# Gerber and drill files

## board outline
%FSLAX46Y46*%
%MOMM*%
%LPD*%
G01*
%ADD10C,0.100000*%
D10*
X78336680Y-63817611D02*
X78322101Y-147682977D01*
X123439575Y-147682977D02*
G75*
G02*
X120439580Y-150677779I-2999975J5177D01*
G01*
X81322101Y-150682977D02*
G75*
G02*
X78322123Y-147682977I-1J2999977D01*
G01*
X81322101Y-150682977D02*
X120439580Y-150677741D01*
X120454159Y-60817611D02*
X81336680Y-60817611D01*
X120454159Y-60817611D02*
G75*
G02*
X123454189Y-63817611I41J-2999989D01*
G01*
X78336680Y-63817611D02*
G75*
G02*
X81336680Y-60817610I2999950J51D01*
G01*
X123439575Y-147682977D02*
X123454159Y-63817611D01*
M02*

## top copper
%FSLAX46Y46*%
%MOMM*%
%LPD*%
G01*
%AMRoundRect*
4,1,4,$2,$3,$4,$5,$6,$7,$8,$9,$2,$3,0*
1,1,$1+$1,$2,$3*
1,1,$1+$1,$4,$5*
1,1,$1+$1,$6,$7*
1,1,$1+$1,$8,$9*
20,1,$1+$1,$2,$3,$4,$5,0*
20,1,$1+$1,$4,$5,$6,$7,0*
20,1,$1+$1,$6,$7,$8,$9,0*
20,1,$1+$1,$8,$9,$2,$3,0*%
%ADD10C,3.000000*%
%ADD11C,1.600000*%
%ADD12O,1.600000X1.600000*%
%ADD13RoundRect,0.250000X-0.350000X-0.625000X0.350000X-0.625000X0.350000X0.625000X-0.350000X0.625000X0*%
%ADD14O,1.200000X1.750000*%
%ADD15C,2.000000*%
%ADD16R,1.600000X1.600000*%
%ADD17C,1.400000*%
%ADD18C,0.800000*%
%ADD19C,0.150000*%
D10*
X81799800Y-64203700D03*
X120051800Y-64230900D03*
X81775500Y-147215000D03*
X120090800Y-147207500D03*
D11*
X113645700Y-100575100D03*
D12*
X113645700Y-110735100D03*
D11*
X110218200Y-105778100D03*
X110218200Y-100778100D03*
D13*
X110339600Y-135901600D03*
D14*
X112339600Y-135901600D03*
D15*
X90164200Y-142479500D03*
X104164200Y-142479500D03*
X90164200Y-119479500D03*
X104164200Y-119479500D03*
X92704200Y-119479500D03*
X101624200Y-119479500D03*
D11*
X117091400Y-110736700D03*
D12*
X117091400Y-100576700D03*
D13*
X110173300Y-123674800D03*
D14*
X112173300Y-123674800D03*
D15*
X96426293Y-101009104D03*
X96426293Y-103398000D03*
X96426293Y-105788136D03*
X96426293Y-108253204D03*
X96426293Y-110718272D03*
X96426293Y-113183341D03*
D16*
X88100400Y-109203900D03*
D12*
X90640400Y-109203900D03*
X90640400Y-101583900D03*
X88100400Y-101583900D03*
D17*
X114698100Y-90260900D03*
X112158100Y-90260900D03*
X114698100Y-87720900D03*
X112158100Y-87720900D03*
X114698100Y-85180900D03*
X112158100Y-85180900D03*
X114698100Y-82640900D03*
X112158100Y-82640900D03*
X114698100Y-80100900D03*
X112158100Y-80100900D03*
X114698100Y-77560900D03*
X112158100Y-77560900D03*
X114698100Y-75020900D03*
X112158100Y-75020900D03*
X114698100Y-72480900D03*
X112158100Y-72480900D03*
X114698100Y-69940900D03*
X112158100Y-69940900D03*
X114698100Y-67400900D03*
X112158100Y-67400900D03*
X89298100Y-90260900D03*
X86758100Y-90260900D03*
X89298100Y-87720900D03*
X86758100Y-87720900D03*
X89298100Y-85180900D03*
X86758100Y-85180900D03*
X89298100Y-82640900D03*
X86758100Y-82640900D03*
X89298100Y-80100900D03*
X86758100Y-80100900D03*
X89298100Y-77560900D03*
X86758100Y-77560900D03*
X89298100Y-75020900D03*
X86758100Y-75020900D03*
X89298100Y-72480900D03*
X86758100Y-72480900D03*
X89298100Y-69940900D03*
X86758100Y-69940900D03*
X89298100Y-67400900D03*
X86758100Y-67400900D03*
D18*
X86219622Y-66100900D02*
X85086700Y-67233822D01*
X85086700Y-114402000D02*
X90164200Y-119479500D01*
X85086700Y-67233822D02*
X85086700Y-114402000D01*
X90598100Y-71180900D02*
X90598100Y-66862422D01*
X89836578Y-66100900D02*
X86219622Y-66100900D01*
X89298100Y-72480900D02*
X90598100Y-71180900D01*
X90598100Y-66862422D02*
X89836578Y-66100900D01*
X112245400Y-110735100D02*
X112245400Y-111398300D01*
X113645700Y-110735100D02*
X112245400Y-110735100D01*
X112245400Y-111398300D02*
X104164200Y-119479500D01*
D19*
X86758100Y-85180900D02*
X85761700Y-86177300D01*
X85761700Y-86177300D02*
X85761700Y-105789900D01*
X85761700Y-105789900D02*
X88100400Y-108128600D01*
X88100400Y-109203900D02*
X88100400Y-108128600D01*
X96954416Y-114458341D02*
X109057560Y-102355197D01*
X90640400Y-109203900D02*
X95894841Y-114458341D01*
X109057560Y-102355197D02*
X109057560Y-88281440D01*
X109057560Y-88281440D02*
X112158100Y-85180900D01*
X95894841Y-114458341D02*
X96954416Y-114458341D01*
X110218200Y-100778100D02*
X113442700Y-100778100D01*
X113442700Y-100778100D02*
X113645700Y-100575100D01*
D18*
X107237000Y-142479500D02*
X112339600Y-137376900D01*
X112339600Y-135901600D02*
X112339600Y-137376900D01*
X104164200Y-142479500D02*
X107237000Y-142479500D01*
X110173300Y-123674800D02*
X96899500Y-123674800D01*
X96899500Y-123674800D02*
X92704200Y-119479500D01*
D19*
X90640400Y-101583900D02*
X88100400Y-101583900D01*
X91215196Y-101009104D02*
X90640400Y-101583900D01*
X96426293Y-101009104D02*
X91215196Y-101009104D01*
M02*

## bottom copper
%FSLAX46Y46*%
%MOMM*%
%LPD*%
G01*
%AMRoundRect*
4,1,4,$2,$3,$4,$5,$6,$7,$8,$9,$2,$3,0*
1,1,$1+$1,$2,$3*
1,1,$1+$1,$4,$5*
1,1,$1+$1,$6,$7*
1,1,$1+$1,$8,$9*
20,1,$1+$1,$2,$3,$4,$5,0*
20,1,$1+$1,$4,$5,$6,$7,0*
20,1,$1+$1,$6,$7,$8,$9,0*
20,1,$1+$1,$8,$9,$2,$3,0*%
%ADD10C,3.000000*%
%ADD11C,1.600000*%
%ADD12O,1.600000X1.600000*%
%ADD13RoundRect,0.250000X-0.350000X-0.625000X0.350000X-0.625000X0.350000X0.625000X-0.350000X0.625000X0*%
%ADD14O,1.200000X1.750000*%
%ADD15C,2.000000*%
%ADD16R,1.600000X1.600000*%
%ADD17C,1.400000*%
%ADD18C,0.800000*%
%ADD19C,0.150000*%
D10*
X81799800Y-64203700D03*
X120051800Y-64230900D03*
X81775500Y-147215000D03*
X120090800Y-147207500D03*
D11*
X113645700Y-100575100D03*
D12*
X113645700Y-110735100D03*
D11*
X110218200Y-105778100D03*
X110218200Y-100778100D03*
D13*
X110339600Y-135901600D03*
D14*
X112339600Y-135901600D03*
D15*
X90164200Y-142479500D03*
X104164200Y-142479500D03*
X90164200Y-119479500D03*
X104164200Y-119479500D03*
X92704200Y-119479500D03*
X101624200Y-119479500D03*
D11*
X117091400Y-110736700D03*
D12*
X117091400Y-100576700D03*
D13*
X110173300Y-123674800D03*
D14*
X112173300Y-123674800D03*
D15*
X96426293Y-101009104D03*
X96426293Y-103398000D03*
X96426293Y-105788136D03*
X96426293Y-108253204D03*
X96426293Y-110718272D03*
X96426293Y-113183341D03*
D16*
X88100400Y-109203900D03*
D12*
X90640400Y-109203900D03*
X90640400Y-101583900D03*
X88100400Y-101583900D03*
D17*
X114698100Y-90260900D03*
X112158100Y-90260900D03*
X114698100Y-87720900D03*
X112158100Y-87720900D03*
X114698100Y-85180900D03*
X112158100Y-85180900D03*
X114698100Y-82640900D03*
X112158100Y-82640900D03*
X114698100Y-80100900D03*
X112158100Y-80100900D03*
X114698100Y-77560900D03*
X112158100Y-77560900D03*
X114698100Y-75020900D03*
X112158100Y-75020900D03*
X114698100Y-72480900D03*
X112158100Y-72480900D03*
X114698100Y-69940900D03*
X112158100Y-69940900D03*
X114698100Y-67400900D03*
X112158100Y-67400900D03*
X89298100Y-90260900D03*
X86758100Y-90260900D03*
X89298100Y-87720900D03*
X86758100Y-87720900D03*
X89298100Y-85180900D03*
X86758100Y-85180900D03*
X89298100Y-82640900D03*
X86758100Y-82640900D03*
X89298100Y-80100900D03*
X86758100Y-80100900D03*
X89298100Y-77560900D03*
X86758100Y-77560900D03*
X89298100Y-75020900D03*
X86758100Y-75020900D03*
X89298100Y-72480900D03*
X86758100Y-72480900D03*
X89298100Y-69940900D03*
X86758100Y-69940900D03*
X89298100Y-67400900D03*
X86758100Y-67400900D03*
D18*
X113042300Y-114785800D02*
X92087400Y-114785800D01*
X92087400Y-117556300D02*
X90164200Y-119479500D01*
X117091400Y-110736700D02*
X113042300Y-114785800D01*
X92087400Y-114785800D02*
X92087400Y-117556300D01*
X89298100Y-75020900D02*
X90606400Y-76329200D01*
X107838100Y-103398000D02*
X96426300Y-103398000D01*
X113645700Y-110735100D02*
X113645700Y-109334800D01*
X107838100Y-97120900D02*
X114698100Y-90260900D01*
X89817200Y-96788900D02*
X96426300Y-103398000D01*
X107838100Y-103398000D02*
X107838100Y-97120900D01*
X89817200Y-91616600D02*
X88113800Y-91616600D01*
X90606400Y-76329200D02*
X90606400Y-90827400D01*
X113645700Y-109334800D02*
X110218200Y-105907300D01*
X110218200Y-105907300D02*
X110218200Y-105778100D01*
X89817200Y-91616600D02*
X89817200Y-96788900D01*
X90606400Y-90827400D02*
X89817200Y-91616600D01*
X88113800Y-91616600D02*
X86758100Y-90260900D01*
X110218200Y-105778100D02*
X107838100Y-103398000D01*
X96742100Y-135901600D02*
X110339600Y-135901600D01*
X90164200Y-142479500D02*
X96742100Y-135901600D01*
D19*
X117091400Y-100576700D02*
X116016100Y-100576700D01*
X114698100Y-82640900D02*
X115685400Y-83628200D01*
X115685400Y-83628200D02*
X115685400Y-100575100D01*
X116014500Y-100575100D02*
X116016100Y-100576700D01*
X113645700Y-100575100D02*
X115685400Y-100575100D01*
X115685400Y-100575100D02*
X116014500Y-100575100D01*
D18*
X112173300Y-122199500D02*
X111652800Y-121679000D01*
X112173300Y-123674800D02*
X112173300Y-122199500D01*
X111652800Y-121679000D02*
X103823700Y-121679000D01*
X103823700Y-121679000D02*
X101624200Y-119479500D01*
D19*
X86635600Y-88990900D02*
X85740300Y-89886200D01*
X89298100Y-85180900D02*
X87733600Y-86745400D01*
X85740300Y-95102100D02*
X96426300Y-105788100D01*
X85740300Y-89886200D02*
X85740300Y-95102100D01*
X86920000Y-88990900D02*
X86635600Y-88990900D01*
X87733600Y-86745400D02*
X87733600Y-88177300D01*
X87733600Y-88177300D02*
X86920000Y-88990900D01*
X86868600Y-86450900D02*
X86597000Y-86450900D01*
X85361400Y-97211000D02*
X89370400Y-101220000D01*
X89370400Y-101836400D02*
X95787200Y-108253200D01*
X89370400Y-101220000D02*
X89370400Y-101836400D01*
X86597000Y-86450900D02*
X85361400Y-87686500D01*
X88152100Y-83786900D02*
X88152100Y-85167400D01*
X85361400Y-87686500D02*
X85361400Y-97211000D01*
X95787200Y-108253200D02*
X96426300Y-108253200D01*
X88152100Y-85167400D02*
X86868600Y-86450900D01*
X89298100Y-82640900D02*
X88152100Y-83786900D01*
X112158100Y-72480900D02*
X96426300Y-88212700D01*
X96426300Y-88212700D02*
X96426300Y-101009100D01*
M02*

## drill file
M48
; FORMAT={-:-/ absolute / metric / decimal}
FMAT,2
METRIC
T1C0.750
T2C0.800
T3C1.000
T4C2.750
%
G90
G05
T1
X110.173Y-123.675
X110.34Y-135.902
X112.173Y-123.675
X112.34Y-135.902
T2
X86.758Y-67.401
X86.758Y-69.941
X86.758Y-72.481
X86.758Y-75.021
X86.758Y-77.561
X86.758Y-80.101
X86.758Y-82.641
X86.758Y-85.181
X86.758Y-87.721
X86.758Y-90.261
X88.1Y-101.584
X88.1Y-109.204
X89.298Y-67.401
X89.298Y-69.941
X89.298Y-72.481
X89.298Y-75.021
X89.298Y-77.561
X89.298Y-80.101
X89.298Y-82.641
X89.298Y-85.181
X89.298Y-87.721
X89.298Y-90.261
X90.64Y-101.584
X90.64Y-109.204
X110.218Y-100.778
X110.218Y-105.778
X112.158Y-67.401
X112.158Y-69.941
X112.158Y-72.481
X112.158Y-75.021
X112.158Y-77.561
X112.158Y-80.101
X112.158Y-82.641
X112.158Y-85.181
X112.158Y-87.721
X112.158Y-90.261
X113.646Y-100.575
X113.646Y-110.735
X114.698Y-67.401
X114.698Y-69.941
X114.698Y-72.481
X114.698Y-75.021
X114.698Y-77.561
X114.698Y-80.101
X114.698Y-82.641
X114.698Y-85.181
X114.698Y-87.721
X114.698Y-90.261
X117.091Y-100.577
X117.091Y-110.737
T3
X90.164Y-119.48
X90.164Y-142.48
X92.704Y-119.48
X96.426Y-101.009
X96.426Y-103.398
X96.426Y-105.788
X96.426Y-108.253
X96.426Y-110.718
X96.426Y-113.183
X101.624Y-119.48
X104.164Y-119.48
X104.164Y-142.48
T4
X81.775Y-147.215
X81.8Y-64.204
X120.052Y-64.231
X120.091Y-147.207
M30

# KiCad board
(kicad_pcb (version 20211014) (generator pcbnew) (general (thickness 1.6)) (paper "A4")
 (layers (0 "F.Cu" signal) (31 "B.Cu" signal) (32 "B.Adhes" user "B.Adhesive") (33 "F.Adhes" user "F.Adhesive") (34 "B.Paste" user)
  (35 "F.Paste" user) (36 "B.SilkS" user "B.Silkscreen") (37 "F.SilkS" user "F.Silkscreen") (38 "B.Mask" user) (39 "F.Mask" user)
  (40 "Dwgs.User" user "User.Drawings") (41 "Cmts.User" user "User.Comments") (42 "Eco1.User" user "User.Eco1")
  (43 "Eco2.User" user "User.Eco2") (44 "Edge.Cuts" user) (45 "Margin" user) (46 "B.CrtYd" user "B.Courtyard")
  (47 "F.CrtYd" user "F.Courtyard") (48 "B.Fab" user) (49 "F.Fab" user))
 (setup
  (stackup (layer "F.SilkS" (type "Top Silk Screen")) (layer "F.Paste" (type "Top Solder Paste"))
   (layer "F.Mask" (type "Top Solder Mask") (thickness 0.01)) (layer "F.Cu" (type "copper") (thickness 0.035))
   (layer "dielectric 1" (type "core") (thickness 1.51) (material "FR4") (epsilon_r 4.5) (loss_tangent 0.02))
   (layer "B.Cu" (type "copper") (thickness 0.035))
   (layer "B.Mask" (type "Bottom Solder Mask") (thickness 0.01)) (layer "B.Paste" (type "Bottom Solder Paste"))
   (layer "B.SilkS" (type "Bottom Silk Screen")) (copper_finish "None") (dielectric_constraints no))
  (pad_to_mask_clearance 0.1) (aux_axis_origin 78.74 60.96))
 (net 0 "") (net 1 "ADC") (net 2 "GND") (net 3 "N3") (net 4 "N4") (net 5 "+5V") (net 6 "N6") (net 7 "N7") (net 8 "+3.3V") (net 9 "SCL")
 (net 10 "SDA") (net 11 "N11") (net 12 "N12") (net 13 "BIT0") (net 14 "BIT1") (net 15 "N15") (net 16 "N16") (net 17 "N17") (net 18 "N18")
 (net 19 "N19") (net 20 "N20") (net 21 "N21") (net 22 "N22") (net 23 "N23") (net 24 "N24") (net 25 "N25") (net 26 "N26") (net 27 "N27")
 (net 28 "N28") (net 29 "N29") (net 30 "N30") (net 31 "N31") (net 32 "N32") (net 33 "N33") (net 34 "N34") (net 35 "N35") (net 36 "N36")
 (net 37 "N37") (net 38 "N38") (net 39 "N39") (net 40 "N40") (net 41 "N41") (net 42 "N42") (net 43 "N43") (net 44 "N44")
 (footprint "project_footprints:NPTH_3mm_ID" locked (layer "F.Cu") (at 81.7998 64.2037)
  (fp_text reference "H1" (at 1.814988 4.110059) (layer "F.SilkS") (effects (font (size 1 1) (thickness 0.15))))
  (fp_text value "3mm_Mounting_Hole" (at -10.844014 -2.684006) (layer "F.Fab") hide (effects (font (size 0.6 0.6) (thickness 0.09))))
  (pad "" np_thru_hole circle locked (at 0 0) (size 3 3) (drill 2.75) (layers *.Cu *.Mask) (clearance 1.6)))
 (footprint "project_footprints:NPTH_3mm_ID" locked (layer "F.Cu") (at 120.0518 64.2309)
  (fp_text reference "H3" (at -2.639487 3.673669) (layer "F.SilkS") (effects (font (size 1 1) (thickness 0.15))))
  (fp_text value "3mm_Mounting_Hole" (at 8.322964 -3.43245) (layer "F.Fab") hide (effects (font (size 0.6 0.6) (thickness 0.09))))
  (pad "" np_thru_hole circle locked (at 0 0) (size 3 3) (drill 2.75) (layers *.Cu *.Mask) (clearance 1.6)))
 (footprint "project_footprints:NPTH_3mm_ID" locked (layer "F.Cu") (at 81.7755 147.215)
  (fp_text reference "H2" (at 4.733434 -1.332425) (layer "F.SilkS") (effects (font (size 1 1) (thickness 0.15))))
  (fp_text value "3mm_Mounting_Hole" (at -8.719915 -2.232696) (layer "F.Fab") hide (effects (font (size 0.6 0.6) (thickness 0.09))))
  (pad "" np_thru_hole circle locked (at 0 0) (size 3 3) (drill 2.75) (layers *.Cu *.Mask) (clearance 1.6)))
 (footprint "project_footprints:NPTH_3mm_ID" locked (layer "F.Cu") (at 120.0908 147.2075)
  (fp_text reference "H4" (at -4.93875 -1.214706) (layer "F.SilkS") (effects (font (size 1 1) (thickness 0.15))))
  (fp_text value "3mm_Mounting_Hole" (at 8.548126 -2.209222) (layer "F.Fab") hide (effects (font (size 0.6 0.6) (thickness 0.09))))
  (pad "" np_thru_hole circle locked (at 0 0) (size 3 3) (drill 2.75) (layers *.Cu *.Mask) (clearance 1.6)))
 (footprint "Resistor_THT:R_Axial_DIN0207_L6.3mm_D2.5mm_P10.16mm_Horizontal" (layer "F.Cu") (at 113.6457 100.5751 -90)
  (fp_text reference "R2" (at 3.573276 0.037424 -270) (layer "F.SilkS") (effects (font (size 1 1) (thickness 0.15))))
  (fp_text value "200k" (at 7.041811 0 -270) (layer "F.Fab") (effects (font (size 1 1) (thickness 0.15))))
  (pad "1" thru_hole circle (at 0 0 270) (size 1.6 1.6) (drill 0.8) (layers *.Cu *.Mask) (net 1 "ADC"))
  (pad "2" thru_hole oval (at 10.16 0 270) (size 1.6 1.6) (drill 0.8) (layers *.Cu *.Mask) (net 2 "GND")))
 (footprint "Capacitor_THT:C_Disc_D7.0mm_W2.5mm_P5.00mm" (layer "F.Cu") (at 110.2182 105.7781 90)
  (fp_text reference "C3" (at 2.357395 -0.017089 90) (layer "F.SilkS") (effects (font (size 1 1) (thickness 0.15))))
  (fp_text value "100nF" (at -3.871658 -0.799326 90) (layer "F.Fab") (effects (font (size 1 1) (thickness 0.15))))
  (pad "1" thru_hole circle (at 0 0 90) (size 1.6 1.6) (drill 0.8) (layers *.Cu *.Mask) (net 2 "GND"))
  (pad "2" thru_hole circle (at 5 0 90) (size 1.6 1.6) (drill 0.8) (layers *.Cu *.Mask) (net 1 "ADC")))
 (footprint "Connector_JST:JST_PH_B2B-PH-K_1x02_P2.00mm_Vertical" (layer "F.Cu") (at 110.3396 135.9016)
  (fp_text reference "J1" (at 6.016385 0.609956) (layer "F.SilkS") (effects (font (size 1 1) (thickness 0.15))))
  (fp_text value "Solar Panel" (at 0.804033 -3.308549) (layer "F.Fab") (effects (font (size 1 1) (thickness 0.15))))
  (pad "1" thru_hole roundrect (at 0 0) (size 1.2 1.75) (drill 0.75) (layers *.Cu *.Mask) (roundrect_rratio 0.208333) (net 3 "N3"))
  (pad "2" thru_hole oval (at 2 0) (size 1.2 1.75) (drill 0.75) (layers *.Cu *.Mask) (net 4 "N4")))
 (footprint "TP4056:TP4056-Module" (layer "F.Cu") (at 105.7642 144.9795 90)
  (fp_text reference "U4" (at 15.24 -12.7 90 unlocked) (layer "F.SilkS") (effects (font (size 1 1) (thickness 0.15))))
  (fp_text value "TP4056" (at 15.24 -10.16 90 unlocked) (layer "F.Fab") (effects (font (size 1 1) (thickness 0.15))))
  (pad "1" thru_hole circle (at 2.5 -15.6 90) (size 2 2) (drill 1) (layers *.Cu *.Mask) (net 3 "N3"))
  (pad "2" thru_hole circle (at 2.5 -1.6 90) (size 2 2) (drill 1) (layers *.Cu *.Mask) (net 4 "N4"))
  (pad "3" thru_hole circle (at 25.5 -15.6 90) (size 2 2) (drill 1) (layers *.Cu *.Mask) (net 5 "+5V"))
  (pad "4" thru_hole circle (at 25.5 -1.6 90) (size 2 2) (drill 1) (layers *.Cu *.Mask) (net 2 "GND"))
  (pad "5" thru_hole circle (at 25.5 -13.06 90) (size 2 2) (drill 1) (layers *.Cu *.Mask) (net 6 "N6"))
  (pad "6" thru_hole circle (at 25.5 -4.14 90) (size 2 2) (drill 1) (layers *.Cu *.Mask) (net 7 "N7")))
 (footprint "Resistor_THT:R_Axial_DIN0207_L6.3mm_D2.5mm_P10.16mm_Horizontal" (layer "F.Cu") (at 117.0914 110.7367 90)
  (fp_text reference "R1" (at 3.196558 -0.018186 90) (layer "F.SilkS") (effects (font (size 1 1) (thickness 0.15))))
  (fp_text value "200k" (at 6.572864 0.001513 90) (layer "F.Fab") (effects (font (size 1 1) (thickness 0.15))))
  (pad "1" thru_hole circle (at 0 0 90) (size 1.6 1.6) (drill 0.8) (layers *.Cu *.Mask) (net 5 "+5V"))
  (pad "2" thru_hole oval (at 10.16 0 90) (size 1.6 1.6) (drill 0.8) (layers *.Cu *.Mask) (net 1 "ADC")))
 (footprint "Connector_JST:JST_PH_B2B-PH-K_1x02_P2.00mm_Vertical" (layer "F.Cu") (at 110.1733 123.6748)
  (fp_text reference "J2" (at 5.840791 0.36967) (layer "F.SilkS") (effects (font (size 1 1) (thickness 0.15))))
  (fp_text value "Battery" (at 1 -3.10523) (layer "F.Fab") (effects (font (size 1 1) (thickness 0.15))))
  (pad "1" thru_hole roundrect (at 0 0) (size 1.2 1.75) (drill 0.75) (layers *.Cu *.Mask) (roundrect_rratio 0.208333) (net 6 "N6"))
  (pad "2" thru_hole oval (at 2 0) (size 1.2 1.75) (drill 0.75) (layers *.Cu *.Mask) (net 7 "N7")))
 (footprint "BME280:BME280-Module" (layer "F.Cu") (at 94.9375 114.558)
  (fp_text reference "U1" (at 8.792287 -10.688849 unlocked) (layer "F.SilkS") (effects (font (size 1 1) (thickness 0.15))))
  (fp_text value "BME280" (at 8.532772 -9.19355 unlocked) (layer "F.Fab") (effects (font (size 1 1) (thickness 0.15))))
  (pad "1" thru_hole circle (at 1.488793 -13.548896) (size 2 2) (drill 1) (layers *.Cu *.Mask) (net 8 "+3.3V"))
  (pad "2" thru_hole circle (at 1.488793 -11.16) (size 2 2) (drill 1) (layers *.Cu *.Mask) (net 2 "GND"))
  (pad "3" thru_hole circle (at 1.488793 -8.769864) (size 2 2) (drill 1) (layers *.Cu *.Mask) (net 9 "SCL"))
  (pad "4" thru_hole circle (at 1.488793 -6.304796) (size 2 2) (drill 1) (layers *.Cu *.Mask) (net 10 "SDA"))
  (pad "5" thru_hole circle (at 1.488793 -3.839728) (size 2 2) (drill 1) (layers *.Cu *.Mask) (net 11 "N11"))
  (pad "6" thru_hole circle (at 1.488793 -1.374659) (size 2 2) (drill 1) (layers *.Cu *.Mask) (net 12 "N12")))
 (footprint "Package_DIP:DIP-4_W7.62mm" (layer "F.Cu") (at 88.1004 109.2039 90)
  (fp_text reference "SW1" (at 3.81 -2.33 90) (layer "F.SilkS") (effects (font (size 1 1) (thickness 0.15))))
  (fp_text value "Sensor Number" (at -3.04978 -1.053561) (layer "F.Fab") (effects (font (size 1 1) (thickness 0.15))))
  (pad "1" thru_hole rect (at 0 0 90) (size 1.6 1.6) (drill 0.8) (layers *.Cu *.Mask) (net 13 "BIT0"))
  (pad "2" thru_hole oval (at 0 2.54 90) (size 1.6 1.6) (drill 0.8) (layers *.Cu *.Mask) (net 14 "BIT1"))
  (pad "3" thru_hole oval (at 7.62 2.54 90) (size 1.6 1.6) (drill 0.8) (layers *.Cu *.Mask) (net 8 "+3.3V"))
  (pad "4" thru_hole oval (at 7.62 0 90) (size 1.6 1.6) (drill 0.8) (layers *.Cu *.Mask) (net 8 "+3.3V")))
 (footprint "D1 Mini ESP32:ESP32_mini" (layer "F.Cu") (at 100.7281 78.8309 180)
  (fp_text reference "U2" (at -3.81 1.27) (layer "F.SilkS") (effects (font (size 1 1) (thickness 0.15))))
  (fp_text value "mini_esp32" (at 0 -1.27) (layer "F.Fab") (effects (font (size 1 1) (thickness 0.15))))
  (pad "1" thru_hole circle locked (at -13.97 -11.43 90) (size 1.4 1.4) (drill 0.8) (layers *.Cu *.Mask) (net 2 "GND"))
  (pad "2" thru_hole circle locked (at -11.43 -11.43 90) (size 1.4 1.4) (drill 0.8) (layers *.Cu *.Mask) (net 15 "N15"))
  (pad "3" thru_hole circle locked (at -13.97 -8.89 90) (size 1.4 1.4) (drill 0.8) (layers *.Cu *.Mask) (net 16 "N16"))
  (pad "4" thru_hole circle locked (at -11.43 -8.89 90) (size 1.4 1.4) (drill 0.8) (layers *.Cu *.Mask) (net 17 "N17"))
  (pad "5" thru_hole circle locked (at -13.97 -6.35 90) (size 1.4 1.4) (drill 0.8) (layers *.Cu *.Mask) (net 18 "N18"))
  (pad "6" thru_hole circle locked (at -11.43 -6.35 90) (size 1.4 1.4) (drill 0.8) (layers *.Cu *.Mask) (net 14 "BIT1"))
  (pad "7" thru_hole circle locked (at -13.97 -3.81 90) (size 1.4 1.4) (drill 0.8) (layers *.Cu *.Mask) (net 1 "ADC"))
  (pad "8" thru_hole circle locked (at -11.43 -3.81 90) (size 1.4 1.4) (drill 0.8) (layers *.Cu *.Mask) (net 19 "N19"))
  (pad "9" thru_hole circle locked (at -13.97 -1.27 90) (size 1.4 1.4) (drill 0.8) (layers *.Cu *.Mask) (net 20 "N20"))
  (pad "10" thru_hole circle locked (at -11.43 -1.27 90) (size 1.4 1.4) (drill 0.8) (layers *.Cu *.Mask) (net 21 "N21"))
  (pad "11" thru_hole circle locked (at -13.97 1.27 90) (size 1.4 1.4) (drill 0.8) (layers *.Cu *.Mask) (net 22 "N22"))
  (pad "12" thru_hole circle locked (at -11.43 1.27 90) (size 1.4 1.4) (drill 0.8) (layers *.Cu *.Mask) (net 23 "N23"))
  (pad "13" thru_hole circle locked (at -13.97 3.81 90) (size 1.4 1.4) (drill 0.8) (layers *.Cu *.Mask) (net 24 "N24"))
  (pad "14" thru_hole circle locked (at -11.43 3.81 90) (size 1.4 1.4) (drill 0.8) (layers *.Cu *.Mask) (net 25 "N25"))
  (pad "15" thru_hole circle locked (at -13.97 6.35 90) (size 1.4 1.4) (drill 0.8) (layers *.Cu *.Mask) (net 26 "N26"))
  (pad "16" thru_hole circle locked (at -11.43 6.35 90) (size 1.4 1.4) (drill 0.8) (layers *.Cu *.Mask) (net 8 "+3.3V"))
  (pad "17" thru_hole circle locked (at -13.97 8.89 90) (size 1.4 1.4) (drill 0.8) (layers *.Cu *.Mask) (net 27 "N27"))
  (pad "18" thru_hole circle locked (at -11.43 8.89 90) (size 1.4 1.4) (drill 0.8) (layers *.Cu *.Mask) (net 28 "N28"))
  (pad "19" thru_hole circle locked (at -13.97 11.43 90) (size 1.4 1.4) (drill 0.8) (layers *.Cu *.Mask) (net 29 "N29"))
  (pad "20" thru_hole circle locked (at -11.43 11.43 90) (size 1.4 1.4) (drill 0.8) (layers *.Cu *.Mask) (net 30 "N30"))
  (pad "21" thru_hole circle locked (at 11.43 -11.43 90) (size 1.4 1.4) (drill 0.8) (layers *.Cu *.Mask) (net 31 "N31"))
  (pad "22" thru_hole circle locked (at 13.97 -11.43 90) (size 1.4 1.4) (drill 0.8) (layers *.Cu *.Mask) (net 2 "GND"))
  (pad "23" thru_hole circle locked (at 11.43 -8.89 90) (size 1.4 1.4) (drill 0.8) (layers *.Cu *.Mask) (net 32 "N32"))
  (pad "24" thru_hole circle locked (at 13.97 -8.89 90) (size 1.4 1.4) (drill 0.8) (layers *.Cu *.Mask) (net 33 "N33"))
  (pad "25" thru_hole circle locked (at 11.43 -6.35 90) (size 1.4 1.4) (drill 0.8) (layers *.Cu *.Mask) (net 9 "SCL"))
  (pad "26" thru_hole circle locked (at 13.97 -6.35 90) (size 1.4 1.4) (drill 0.8) (layers *.Cu *.Mask) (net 13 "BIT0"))
  (pad "27" thru_hole circle locked (at 11.43 -3.81 90) (size 1.4 1.4) (drill 0.8) (layers *.Cu *.Mask) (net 10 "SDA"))
  (pad "28" thru_hole circle locked (at 13.97 -3.81 90) (size 1.4 1.4) (drill 0.8) (layers *.Cu *.Mask) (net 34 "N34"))
  (pad "29" thru_hole circle locked (at 11.43 -1.27 90) (size 1.4 1.4) (drill 0.8) (layers *.Cu *.Mask) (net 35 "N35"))
  (pad "30" thru_hole circle locked (at 13.97 -1.27 90) (size 1.4 1.4) (drill 0.8) (layers *.Cu *.Mask) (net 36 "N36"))
  (pad "31" thru_hole circle locked (at 11.43 1.27 90) (size 1.4 1.4) (drill 0.8) (layers *.Cu *.Mask) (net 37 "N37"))
  (pad "32" thru_hole circle locked (at 13.97 1.27 90) (size 1.4 1.4) (drill 0.8) (layers *.Cu *.Mask) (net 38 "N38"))
  (pad "33" thru_hole circle locked (at 11.43 3.81 90) (size 1.4 1.4) (drill 0.8) (layers *.Cu *.Mask) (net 2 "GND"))
  (pad "34" thru_hole circle locked (at 13.97 3.81 90) (size 1.4 1.4) (drill 0.8) (layers *.Cu *.Mask) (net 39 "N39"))
  (pad "35" thru_hole circle locked (at 11.43 6.35 90) (size 1.4 1.4) (drill 0.8) (layers *.Cu *.Mask) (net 5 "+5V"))
  (pad "36" thru_hole circle locked (at 13.97 6.35 90) (size 1.4 1.4) (drill 0.8) (layers *.Cu *.Mask) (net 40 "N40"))
  (pad "37" thru_hole circle locked (at 11.43 8.89 90) (size 1.4 1.4) (drill 0.8) (layers *.Cu *.Mask) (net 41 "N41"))
  (pad "38" thru_hole circle locked (at 13.97 8.89 90) (size 1.4 1.4) (drill 0.8) (layers *.Cu *.Mask) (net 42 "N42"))
  (pad "39" thru_hole circle locked (at 11.43 11.43 90) (size 1.4 1.4) (drill 0.8) (layers *.Cu *.Mask) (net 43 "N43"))
  (pad "40" thru_hole circle locked (at 13.97 11.43 90) (size 1.4 1.4) (drill 0.8) (layers *.Cu *.Mask) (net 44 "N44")))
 (gr_line (start 78.33668 63.817611) (end 78.322101 147.682977) (layer "Edge.Cuts") (width 0.1))
 (gr_arc (start 123.439575 147.682977) (mid 122.559047 149.80092) (end 120.43958 150.677741) (layer "Edge.Cuts") (width 0.1))
 (gr_arc (start 81.322101 150.682977) (mid 79.200777 149.804293) (end 78.322101 147.682977) (layer "Edge.Cuts") (width 0.1))
 (gr_line (start 81.322101 150.682977) (end 120.43958 150.677741) (layer "Edge.Cuts") (width 0.1))
 (gr_line (start 120.454159 60.817611) (end 81.33668 60.817611) (layer "Edge.Cuts") (width 0.1))
 (gr_arc (start 120.454159 60.817611) (mid 122.575479 61.696276) (end 123.454159 63.817611) (layer "Edge.Cuts") (width 0.1))
 (gr_arc (start 78.33668 63.817611) (mid 79.215353 61.696268) (end 81.33668 60.817611) (layer "Edge.Cuts") (width 0.1))
 (gr_line (start 123.439575 147.682977) (end 123.454159 63.817611) (layer "Edge.Cuts") (width 0.1))
 (segment (start 86.219622 66.1009) (end 85.0867 67.233822) (width 0.8) (layer "F.Cu") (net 5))
 (segment (start 85.0867 114.402) (end 90.1642 119.4795) (width 0.8) (layer "F.Cu") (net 5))
 (segment (start 85.0867 67.233822) (end 85.0867 114.402) (width 0.8) (layer "F.Cu") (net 5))
 (segment (start 90.5981 71.1809) (end 90.5981 66.862422) (width 0.8) (layer "F.Cu") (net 5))
 (segment (start 89.836578 66.1009) (end 86.219622 66.1009) (width 0.8) (layer "F.Cu") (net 5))
 (segment (start 89.2981 72.4809) (end 90.5981 71.1809) (width 0.8) (layer "F.Cu") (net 5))
 (segment (start 90.5981 66.862422) (end 89.836578 66.1009) (width 0.8) (layer "F.Cu") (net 5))
 (segment (start 113.0423 114.7858) (end 92.0874 114.7858) (width 0.8) (layer "B.Cu") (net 5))
 (segment (start 92.0874 117.5563) (end 90.1642 119.4795) (width 0.8) (layer "B.Cu") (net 5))
 (segment (start 117.0914 110.7367) (end 113.0423 114.7858) (width 0.8) (layer "B.Cu") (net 5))
 (segment (start 92.0874 114.7858) (end 92.0874 117.5563) (width 0.8) (layer "B.Cu") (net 5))
 (segment (start 112.2454 110.7351) (end 112.2454 111.3983) (width 0.8) (layer "F.Cu") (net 2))
 (segment (start 113.6457 110.7351) (end 112.2454 110.7351) (width 0.8) (layer "F.Cu") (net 2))
 (segment (start 112.2454 111.3983) (end 104.1642 119.4795) (width 0.8) (layer "F.Cu") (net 2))
 (segment (start 89.2981 75.0209) (end 90.6064 76.3292) (width 0.8) (layer "B.Cu") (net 2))
 (segment (start 107.8381 103.398) (end 96.4263 103.398) (width 0.8) (layer "B.Cu") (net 2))
 (segment (start 113.6457 110.7351) (end 113.6457 109.3348) (width 0.8) (layer "B.Cu") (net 2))
 (segment (start 107.8381 97.1209) (end 114.6981 90.2609) (width 0.8) (layer "B.Cu") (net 2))
 (segment (start 89.8172 96.7889) (end 96.4263 103.398) (width 0.8) (layer "B.Cu") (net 2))
 (segment (start 107.8381 103.398) (end 107.8381 97.1209) (width 0.8) (layer "B.Cu") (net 2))
 (segment (start 89.8172 91.6166) (end 88.1138 91.6166) (width 0.8) (layer "B.Cu") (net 2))
 (segment (start 90.6064 76.3292) (end 90.6064 90.8274) (width 0.8) (layer "B.Cu") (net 2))
 (segment (start 113.6457 109.3348) (end 110.2182 105.9073) (width 0.8) (layer "B.Cu") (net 2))
 (segment (start 110.2182 105.9073) (end 110.2182 105.7781) (width 0.8) (layer "B.Cu") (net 2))
 (segment (start 89.8172 91.6166) (end 89.8172 96.7889) (width 0.8) (layer "B.Cu") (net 2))
 (segment (start 90.6064 90.8274) (end 89.8172 91.6166) (width 0.8) (layer "B.Cu") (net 2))
 (segment (start 88.1138 91.6166) (end 86.7581 90.2609) (width 0.8) (layer "B.Cu") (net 2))
 (segment (start 110.2182 105.7781) (end 107.8381 103.398) (width 0.8) (layer "B.Cu") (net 2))
 (segment (start 86.7581 85.1809) (end 85.7617 86.1773) (width 0.15) (layer "F.Cu") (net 13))
 (segment (start 85.7617 86.1773) (end 85.7617 105.7899) (width 0.15) (layer "F.Cu") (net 13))
 (segment (start 85.7617 105.7899) (end 88.1004 108.1286) (width 0.15) (layer "F.Cu") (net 13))
 (segment (start 88.1004 109.2039) (end 88.1004 108.1286) (width 0.15) (layer "F.Cu") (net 13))
 (segment (start 96.954416 114.458341) (end 109.05756 102.355197) (width 0.15) (layer "F.Cu") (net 14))
 (segment (start 90.6404 109.2039) (end 95.894841 114.458341) (width 0.15) (layer "F.Cu") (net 14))
 (segment (start 109.05756 102.355197) (end 109.05756 88.28144) (width 0.15) (layer "F.Cu") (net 14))
 (segment (start 109.05756 88.28144) (end 112.1581 85.1809) (width 0.15) (layer "F.Cu") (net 14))
 (segment (start 95.894841 114.458341) (end 96.954416 114.458341) (width 0.15) (layer "F.Cu") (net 14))
 (segment (start 96.7421 135.9016) (end 110.3396 135.9016) (width 0.8) (layer "B.Cu") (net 3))
 (segment (start 90.1642 142.4795) (end 96.7421 135.9016) (width 0.8) (layer "B.Cu") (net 3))
 (segment (start 110.2182 100.7781) (end 113.4427 100.7781) (width 0.15) (layer "F.Cu") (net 1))
 (segment (start 113.4427 100.7781) (end 113.6457 100.5751) (width 0.15) (layer "F.Cu") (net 1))
 (segment (start 117.0914 100.5767) (end 116.0161 100.5767) (width 0.15) (layer "B.Cu") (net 1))
 (segment (start 114.6981 82.6409) (end 115.6854 83.6282) (width 0.15) (layer "B.Cu") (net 1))
 (segment (start 115.6854 83.6282) (end 115.6854 100.5751) (width 0.15) (layer "B.Cu") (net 1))
 (segment (start 116.0145 100.5751) (end 116.0161 100.5767) (width 0.15) (layer "B.Cu") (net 1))
 (segment (start 113.6457 100.5751) (end 115.6854 100.5751) (width 0.15) (layer "B.Cu") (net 1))
 (segment (start 115.6854 100.5751) (end 116.0145 100.5751) (width 0.15) (layer "B.Cu") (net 1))
 (segment (start 107.237 142.4795) (end 112.3396 137.3769) (width 0.8) (layer "F.Cu") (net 4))
 (segment (start 112.3396 135.9016) (end 112.3396 137.3769) (width 0.8) (layer "F.Cu") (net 4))
 (segment (start 104.1642 142.4795) (end 107.237 142.4795) (width 0.8) (layer "F.Cu") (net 4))
 (segment (start 110.1733 123.6748) (end 96.8995 123.6748) (width 0.8) (layer "F.Cu") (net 6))
 (segment (start 96.8995 123.6748) (end 92.7042 119.4795) (width 0.8) (layer "F.Cu") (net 6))
 (segment (start 112.1733 122.1995) (end 111.6528 121.679) (width 0.8) (layer "B.Cu") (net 7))
 (segment (start 112.1733 123.6748) (end 112.1733 122.1995) (width 0.8) (layer "B.Cu") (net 7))
 (segment (start 111.6528 121.679) (end 103.8237 121.679) (width 0.8) (layer "B.Cu") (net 7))
 (segment (start 103.8237 121.679) (end 101.6242 119.4795) (width 0.8) (layer "B.Cu") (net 7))
 (segment (start 86.6356 88.9909) (end 85.7403 89.8862) (width 0.15) (layer "B.Cu") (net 9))
 (segment (start 89.2981 85.1809) (end 87.7336 86.7454) (width 0.15) (layer "B.Cu") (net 9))
 (segment (start 85.7403 95.1021) (end 96.4263 105.7881) (width 0.15) (layer "B.Cu") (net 9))
 (segment (start 85.7403 89.8862) (end 85.7403 95.1021) (width 0.15) (layer "B.Cu") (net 9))
 (segment (start 86.92 88.9909) (end 86.6356 88.9909) (width 0.15) (layer "B.Cu") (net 9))
 (segment (start 87.7336 86.7454) (end 87.7336 88.1773) (width 0.15) (layer "B.Cu") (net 9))
 (segment (start 87.7336 88.1773) (end 86.92 88.9909) (width 0.15) (layer "B.Cu") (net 9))
 (segment (start 86.8686 86.4509) (end 86.597 86.4509) (width 0.15) (layer "B.Cu") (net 10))
 (segment (start 85.3614 97.211) (end 89.3704 101.22) (width 0.15) (layer "B.Cu") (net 10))
 (segment (start 89.3704 101.8364) (end 95.7872 108.2532) (width 0.15) (layer "B.Cu") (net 10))
 (segment (start 89.3704 101.22) (end 89.3704 101.8364) (width 0.15) (layer "B.Cu") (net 10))
 (segment (start 86.597 86.4509) (end 85.3614 87.6865) (width 0.15) (layer "B.Cu") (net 10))
 (segment (start 88.1521 83.7869) (end 88.1521 85.1674) (width 0.15) (layer "B.Cu") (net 10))
 (segment (start 85.3614 87.6865) (end 85.3614 97.211) (width 0.15) (layer "B.Cu") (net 10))
 (segment (start 95.7872 108.2532) (end 96.4263 108.2532) (width 0.15) (layer "B.Cu") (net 10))
 (segment (start 88.1521 85.1674) (end 86.8686 86.4509) (width 0.15) (layer "B.Cu") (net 10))
 (segment (start 89.2981 82.6409) (end 88.1521 83.7869) (width 0.15) (layer "B.Cu") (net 10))
 (segment (start 90.6404 101.5839) (end 88.1004 101.5839) (width 0.15) (layer "F.Cu") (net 8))
 (segment (start 91.215196 101.009104) (end 90.6404 101.5839) (width 0.15) (layer "F.Cu") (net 8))
 (segment (start 96.426293 101.009104) (end 91.215196 101.009104) (width 0.15) (layer "F.Cu") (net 8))
 (segment (start 112.1581 72.4809) (end 96.4263 88.2127) (width 0.15) (layer "B.Cu") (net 8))
 (segment (start 96.4263 88.2127) (end 96.4263 101.0091) (width 0.15) (layer "B.Cu") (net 8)))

